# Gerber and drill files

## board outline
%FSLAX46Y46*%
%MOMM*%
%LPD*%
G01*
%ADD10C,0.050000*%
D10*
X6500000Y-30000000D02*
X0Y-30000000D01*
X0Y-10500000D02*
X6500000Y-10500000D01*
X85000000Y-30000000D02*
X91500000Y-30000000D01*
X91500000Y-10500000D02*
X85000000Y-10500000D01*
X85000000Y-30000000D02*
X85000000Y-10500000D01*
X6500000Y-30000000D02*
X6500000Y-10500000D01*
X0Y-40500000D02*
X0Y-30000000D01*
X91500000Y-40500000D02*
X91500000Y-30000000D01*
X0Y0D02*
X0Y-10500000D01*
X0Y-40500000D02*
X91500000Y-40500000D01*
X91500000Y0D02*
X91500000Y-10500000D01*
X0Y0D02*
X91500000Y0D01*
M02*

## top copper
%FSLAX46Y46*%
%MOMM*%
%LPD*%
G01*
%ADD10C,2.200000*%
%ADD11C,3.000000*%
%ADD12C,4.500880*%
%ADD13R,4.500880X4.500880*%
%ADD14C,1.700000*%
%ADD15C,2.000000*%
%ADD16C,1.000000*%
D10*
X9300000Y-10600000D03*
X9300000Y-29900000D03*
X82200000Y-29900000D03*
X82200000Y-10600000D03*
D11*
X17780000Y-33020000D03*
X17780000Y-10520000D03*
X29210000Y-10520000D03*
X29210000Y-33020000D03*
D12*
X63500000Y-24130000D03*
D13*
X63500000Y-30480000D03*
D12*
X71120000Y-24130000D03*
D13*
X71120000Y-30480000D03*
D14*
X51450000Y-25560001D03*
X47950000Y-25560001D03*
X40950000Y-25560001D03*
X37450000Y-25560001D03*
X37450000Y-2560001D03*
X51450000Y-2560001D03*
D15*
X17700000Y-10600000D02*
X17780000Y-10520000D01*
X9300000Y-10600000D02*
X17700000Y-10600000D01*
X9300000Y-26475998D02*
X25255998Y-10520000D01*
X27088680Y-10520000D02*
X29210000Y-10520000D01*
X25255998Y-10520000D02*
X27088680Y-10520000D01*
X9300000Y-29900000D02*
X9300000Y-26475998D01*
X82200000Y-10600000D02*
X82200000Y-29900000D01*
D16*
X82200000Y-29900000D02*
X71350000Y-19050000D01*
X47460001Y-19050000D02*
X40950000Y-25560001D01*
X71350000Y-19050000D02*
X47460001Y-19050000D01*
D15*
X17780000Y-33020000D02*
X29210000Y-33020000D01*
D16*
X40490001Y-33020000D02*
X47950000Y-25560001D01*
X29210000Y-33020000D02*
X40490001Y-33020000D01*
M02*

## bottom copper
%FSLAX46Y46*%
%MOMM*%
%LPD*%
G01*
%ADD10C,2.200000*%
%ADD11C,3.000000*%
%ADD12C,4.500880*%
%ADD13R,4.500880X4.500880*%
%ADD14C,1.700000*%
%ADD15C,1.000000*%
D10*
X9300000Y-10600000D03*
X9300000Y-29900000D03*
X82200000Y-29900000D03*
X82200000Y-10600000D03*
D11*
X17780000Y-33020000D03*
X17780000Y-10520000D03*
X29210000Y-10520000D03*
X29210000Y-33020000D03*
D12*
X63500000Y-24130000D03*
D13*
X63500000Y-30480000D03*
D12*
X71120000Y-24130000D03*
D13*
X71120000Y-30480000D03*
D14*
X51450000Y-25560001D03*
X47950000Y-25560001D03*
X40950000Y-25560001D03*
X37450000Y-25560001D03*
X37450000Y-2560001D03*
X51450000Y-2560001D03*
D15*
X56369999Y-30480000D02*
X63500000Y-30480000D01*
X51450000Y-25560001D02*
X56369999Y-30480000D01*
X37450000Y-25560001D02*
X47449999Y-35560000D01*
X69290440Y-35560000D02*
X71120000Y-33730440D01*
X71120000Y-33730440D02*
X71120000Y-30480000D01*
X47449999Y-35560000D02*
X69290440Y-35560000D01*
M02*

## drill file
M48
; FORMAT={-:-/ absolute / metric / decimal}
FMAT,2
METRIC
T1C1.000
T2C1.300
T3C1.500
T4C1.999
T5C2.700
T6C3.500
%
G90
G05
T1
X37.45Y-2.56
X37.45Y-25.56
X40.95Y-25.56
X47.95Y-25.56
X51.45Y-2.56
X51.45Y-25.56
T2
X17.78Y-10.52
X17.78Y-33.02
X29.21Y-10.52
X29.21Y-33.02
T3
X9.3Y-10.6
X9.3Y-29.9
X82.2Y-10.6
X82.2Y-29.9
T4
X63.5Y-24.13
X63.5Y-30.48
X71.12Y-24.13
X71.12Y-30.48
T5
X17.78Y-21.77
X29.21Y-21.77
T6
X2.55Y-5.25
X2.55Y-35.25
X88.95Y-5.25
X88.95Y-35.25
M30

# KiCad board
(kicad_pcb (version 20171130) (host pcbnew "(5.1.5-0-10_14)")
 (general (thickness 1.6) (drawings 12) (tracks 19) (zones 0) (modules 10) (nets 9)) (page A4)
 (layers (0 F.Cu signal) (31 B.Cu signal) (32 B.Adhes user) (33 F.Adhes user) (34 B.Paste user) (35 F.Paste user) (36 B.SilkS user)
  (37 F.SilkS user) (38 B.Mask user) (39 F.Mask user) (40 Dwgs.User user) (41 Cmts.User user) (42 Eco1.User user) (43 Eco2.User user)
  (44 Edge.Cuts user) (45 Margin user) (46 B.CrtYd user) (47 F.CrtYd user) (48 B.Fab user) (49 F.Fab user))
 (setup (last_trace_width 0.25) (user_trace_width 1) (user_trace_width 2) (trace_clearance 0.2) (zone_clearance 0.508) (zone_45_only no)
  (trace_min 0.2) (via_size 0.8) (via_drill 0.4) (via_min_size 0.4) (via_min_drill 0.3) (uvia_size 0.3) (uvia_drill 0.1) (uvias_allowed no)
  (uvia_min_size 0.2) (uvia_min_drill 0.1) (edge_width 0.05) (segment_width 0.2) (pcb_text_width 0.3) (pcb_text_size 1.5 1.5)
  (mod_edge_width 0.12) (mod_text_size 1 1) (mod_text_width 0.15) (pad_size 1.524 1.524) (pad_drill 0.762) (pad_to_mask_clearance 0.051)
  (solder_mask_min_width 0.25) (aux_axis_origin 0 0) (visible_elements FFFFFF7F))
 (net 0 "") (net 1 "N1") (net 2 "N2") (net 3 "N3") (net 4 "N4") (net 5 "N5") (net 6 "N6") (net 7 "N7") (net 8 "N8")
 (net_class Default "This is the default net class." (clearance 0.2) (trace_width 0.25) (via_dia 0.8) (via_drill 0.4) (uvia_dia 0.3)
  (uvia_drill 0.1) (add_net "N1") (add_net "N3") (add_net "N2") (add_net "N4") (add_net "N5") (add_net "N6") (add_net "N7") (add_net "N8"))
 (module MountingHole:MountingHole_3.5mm (layer F.Cu) (at 88.95 35.25)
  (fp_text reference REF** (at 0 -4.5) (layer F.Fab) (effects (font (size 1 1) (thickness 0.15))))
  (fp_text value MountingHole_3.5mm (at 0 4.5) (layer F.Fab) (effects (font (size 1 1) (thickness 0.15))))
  (pad 1 np_thru_hole circle (at 0 0) (size 3.5 3.5) (drill 3.5) (layers *.Cu *.Mask)))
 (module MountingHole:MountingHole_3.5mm (layer F.Cu) (at 88.95 5.25)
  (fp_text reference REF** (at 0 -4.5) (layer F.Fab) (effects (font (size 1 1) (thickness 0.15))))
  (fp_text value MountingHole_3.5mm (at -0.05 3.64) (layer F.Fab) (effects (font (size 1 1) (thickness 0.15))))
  (pad 1 np_thru_hole circle (at 0 0) (size 3.5 3.5) (drill 3.5) (layers *.Cu *.Mask)))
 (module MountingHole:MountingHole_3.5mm (layer F.Cu) (at 2.55 35.25)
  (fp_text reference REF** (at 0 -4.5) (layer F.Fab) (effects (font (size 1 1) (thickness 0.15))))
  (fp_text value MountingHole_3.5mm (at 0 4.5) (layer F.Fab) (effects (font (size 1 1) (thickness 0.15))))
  (pad 1 np_thru_hole circle (at 0 0) (size 3.5 3.5) (drill 3.5) (layers *.Cu *.Mask)))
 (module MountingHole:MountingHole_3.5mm (layer F.Cu) (at 2.55 5.25)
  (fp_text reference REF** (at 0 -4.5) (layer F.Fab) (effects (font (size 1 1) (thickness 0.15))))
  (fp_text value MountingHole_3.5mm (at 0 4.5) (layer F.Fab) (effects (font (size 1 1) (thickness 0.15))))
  (pad 1 np_thru_hole circle (at 0 0) (size 3.5 3.5) (drill 3.5) (layers *.Cu *.Mask)))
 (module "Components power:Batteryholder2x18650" (layer F.Cu) (at 45.75 20.25)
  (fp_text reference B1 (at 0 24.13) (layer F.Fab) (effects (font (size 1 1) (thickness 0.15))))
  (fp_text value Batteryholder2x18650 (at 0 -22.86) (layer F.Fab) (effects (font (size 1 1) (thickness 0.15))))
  (pad 1 thru_hole circle (at -36.45 -9.65) (size 2.2 2.2) (drill 1.5) (layers *.Cu *.Mask) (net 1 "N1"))
  (pad 3 thru_hole circle (at -36.45 9.65) (size 2.2 2.2) (drill 1.5) (layers *.Cu *.Mask) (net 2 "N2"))
  (pad 4 thru_hole circle (at 36.45 9.65) (size 2.2 2.2) (drill 1.5) (layers *.Cu *.Mask) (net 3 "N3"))
  (pad 2 thru_hole circle (at 36.45 -9.65) (size 2.2 2.2) (drill 1.5) (layers *.Cu *.Mask) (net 3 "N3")))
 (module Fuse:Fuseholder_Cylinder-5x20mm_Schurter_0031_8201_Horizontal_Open (layer F.Cu) (at 17.78 33.02 90)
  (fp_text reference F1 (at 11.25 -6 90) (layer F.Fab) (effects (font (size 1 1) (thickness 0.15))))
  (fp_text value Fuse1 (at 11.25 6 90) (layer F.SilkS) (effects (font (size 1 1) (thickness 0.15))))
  (pad 1 thru_hole circle (at 0 0 90) (size 3 3) (drill 1.3) (layers *.Cu *.Mask) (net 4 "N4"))
  (pad 2 thru_hole circle (at 22.5 0 90) (size 3 3) (drill 1.3) (layers *.Cu *.Mask) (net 1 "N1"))
  (pad "" np_thru_hole circle (at 11.25 0 90) (size 2.7 2.7) (drill 2.7) (layers *.Cu *.Mask)))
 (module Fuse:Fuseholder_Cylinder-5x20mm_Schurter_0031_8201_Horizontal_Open (layer F.Cu) (at 29.21 33.02 90)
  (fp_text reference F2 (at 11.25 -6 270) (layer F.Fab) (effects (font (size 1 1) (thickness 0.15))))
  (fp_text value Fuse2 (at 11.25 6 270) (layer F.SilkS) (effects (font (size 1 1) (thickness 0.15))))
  (pad "" np_thru_hole circle (at 11.25 0 90) (size 2.7 2.7) (drill 2.7) (layers *.Cu *.Mask))
  (pad 2 thru_hole circle (at 22.5 0 90) (size 3 3) (drill 1.3) (layers *.Cu *.Mask) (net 2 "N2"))
  (pad 1 thru_hole circle (at 0 0 90) (size 3 3) (drill 1.3) (layers *.Cu *.Mask) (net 4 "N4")))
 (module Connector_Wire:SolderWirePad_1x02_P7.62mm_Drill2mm (layer F.Cu) (at 63.5 30.48 90)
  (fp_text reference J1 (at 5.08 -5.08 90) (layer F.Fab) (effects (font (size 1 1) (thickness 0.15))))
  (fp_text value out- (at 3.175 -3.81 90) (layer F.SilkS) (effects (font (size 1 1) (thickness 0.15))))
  (pad 2 thru_hole circle (at 6.35 0 90) (size 4.50088 4.50088) (drill 1.99898) (layers *.Cu *.Mask))
  (pad 1 thru_hole rect (at 0 0 90) (size 4.50088 4.50088) (drill 1.99898) (layers *.Cu *.Mask) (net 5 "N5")))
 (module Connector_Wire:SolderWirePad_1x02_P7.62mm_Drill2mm (layer F.Cu) (at 71.12 30.48 90)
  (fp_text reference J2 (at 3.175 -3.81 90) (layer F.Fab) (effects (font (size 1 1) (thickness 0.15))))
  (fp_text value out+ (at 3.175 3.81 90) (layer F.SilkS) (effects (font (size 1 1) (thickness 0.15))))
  (pad 2 thru_hole circle (at 6.35 0 90) (size 4.50088 4.50088) (drill 1.99898) (layers *.Cu *.Mask))
  (pad 1 thru_hole rect (at 0 0 90) (size 4.50088 4.50088) (drill 1.99898) (layers *.Cu *.Mask) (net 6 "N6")))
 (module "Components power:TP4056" (layer F.Cu) (at 44.45 14.060001 180)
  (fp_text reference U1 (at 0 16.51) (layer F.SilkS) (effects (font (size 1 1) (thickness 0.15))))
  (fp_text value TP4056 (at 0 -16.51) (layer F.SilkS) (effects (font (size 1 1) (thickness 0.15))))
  (pad 1 thru_hole circle (at -7 -11.5 180) (size 1.7 1.7) (drill 1) (layers *.Cu *.Mask) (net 5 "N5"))
  (pad 2 thru_hole circle (at -3.5 -11.5 180) (size 1.7 1.7) (drill 1) (layers *.Cu *.Mask) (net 4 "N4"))
  (pad 3 thru_hole circle (at 3.5 -11.5 180) (size 1.7 1.7) (drill 1) (layers *.Cu *.Mask) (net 3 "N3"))
  (pad 4 thru_hole circle (at 7 -11.5 180) (size 1.7 1.7) (drill 1) (layers *.Cu *.Mask) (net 6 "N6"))
  (pad 5 thru_hole circle (at 7 11.5 180) (size 1.7 1.7) (drill 1) (layers *.Cu *.Mask) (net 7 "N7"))
  (pad 6 thru_hole circle (at -7 11.5 180) (size 1.7 1.7) (drill 1) (layers *.Cu *.Mask) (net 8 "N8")))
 (gr_line (start 6.5 30) (end 0 30) (layer Edge.Cuts) (width 0.05))
 (gr_line (start 0 10.5) (end 6.5 10.5) (layer Edge.Cuts) (width 0.05))
 (gr_line (start 85 30) (end 91.5 30) (layer Edge.Cuts) (width 0.05))
 (gr_line (start 91.5 10.5) (end 85 10.5) (layer Edge.Cuts) (width 0.05))
 (gr_line (start 85 30) (end 85 10.5) (layer Edge.Cuts) (width 0.05))
 (gr_line (start 6.5 30) (end 6.5 10.5) (layer Edge.Cuts) (width 0.05))
 (gr_line (start 0 40.5) (end 0 30) (layer Edge.Cuts) (width 0.05))
 (gr_line (start 91.5 40.5) (end 91.5 30) (layer Edge.Cuts) (width 0.05))
 (gr_line (start 0 0) (end 0 10.5) (layer Edge.Cuts) (width 0.05))
 (gr_line (start 0 40.5) (end 91.5 40.5) (layer Edge.Cuts) (width 0.05))
 (gr_line (start 91.5 0) (end 91.5 10.5) (layer Edge.Cuts) (width 0.05))
 (gr_line (start 0 0) (end 91.5 0) (layer Edge.Cuts) (width 0.05))
 (segment (start 17.7 10.6) (end 17.78 10.52) (width 2) (layer F.Cu) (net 1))
 (segment (start 9.3 10.6) (end 17.7 10.6) (width 2) (layer F.Cu) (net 1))
 (segment (start 9.3 26.475998) (end 25.255998 10.52) (width 2) (layer F.Cu) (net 2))
 (segment (start 27.08868 10.52) (end 29.21 10.52) (width 2) (layer F.Cu) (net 2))
 (segment (start 25.255998 10.52) (end 27.08868 10.52) (width 2) (layer F.Cu) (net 2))
 (segment (start 9.3 29.9) (end 9.3 26.475998) (width 2) (layer F.Cu) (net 2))
 (segment (start 82.2 10.6) (end 82.2 29.9) (width 2) (layer F.Cu) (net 3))
 (segment (start 82.2 29.9) (end 71.35 19.05) (width 1) (layer F.Cu) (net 3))
 (segment (start 47.460001 19.05) (end 40.95 25.560001) (width 1) (layer F.Cu) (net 3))
 (segment (start 71.35 19.05) (end 47.460001 19.05) (width 1) (layer F.Cu) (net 3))
 (segment (start 17.78 33.02) (end 29.21 33.02) (width 2) (layer F.Cu) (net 4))
 (segment (start 40.490001 33.02) (end 47.95 25.560001) (width 1) (layer F.Cu) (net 4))
 (segment (start 29.21 33.02) (end 40.490001 33.02) (width 1) (layer F.Cu) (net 4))
 (segment (start 56.369999 30.48) (end 63.5 30.48) (width 1) (layer B.Cu) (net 5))
 (segment (start 51.45 25.560001) (end 56.369999 30.48) (width 1) (layer B.Cu) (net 5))
 (segment (start 37.45 25.560001) (end 47.449999 35.56) (width 1) (layer B.Cu) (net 6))
 (segment (start 69.29044 35.56) (end 71.12 33.73044) (width 1) (layer B.Cu) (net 6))
 (segment (start 71.12 33.73044) (end 71.12 30.48) (width 1) (layer B.Cu) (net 6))
 (segment (start 47.449999 35.56) (end 69.29044 35.56) (width 1) (layer B.Cu) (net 6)))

